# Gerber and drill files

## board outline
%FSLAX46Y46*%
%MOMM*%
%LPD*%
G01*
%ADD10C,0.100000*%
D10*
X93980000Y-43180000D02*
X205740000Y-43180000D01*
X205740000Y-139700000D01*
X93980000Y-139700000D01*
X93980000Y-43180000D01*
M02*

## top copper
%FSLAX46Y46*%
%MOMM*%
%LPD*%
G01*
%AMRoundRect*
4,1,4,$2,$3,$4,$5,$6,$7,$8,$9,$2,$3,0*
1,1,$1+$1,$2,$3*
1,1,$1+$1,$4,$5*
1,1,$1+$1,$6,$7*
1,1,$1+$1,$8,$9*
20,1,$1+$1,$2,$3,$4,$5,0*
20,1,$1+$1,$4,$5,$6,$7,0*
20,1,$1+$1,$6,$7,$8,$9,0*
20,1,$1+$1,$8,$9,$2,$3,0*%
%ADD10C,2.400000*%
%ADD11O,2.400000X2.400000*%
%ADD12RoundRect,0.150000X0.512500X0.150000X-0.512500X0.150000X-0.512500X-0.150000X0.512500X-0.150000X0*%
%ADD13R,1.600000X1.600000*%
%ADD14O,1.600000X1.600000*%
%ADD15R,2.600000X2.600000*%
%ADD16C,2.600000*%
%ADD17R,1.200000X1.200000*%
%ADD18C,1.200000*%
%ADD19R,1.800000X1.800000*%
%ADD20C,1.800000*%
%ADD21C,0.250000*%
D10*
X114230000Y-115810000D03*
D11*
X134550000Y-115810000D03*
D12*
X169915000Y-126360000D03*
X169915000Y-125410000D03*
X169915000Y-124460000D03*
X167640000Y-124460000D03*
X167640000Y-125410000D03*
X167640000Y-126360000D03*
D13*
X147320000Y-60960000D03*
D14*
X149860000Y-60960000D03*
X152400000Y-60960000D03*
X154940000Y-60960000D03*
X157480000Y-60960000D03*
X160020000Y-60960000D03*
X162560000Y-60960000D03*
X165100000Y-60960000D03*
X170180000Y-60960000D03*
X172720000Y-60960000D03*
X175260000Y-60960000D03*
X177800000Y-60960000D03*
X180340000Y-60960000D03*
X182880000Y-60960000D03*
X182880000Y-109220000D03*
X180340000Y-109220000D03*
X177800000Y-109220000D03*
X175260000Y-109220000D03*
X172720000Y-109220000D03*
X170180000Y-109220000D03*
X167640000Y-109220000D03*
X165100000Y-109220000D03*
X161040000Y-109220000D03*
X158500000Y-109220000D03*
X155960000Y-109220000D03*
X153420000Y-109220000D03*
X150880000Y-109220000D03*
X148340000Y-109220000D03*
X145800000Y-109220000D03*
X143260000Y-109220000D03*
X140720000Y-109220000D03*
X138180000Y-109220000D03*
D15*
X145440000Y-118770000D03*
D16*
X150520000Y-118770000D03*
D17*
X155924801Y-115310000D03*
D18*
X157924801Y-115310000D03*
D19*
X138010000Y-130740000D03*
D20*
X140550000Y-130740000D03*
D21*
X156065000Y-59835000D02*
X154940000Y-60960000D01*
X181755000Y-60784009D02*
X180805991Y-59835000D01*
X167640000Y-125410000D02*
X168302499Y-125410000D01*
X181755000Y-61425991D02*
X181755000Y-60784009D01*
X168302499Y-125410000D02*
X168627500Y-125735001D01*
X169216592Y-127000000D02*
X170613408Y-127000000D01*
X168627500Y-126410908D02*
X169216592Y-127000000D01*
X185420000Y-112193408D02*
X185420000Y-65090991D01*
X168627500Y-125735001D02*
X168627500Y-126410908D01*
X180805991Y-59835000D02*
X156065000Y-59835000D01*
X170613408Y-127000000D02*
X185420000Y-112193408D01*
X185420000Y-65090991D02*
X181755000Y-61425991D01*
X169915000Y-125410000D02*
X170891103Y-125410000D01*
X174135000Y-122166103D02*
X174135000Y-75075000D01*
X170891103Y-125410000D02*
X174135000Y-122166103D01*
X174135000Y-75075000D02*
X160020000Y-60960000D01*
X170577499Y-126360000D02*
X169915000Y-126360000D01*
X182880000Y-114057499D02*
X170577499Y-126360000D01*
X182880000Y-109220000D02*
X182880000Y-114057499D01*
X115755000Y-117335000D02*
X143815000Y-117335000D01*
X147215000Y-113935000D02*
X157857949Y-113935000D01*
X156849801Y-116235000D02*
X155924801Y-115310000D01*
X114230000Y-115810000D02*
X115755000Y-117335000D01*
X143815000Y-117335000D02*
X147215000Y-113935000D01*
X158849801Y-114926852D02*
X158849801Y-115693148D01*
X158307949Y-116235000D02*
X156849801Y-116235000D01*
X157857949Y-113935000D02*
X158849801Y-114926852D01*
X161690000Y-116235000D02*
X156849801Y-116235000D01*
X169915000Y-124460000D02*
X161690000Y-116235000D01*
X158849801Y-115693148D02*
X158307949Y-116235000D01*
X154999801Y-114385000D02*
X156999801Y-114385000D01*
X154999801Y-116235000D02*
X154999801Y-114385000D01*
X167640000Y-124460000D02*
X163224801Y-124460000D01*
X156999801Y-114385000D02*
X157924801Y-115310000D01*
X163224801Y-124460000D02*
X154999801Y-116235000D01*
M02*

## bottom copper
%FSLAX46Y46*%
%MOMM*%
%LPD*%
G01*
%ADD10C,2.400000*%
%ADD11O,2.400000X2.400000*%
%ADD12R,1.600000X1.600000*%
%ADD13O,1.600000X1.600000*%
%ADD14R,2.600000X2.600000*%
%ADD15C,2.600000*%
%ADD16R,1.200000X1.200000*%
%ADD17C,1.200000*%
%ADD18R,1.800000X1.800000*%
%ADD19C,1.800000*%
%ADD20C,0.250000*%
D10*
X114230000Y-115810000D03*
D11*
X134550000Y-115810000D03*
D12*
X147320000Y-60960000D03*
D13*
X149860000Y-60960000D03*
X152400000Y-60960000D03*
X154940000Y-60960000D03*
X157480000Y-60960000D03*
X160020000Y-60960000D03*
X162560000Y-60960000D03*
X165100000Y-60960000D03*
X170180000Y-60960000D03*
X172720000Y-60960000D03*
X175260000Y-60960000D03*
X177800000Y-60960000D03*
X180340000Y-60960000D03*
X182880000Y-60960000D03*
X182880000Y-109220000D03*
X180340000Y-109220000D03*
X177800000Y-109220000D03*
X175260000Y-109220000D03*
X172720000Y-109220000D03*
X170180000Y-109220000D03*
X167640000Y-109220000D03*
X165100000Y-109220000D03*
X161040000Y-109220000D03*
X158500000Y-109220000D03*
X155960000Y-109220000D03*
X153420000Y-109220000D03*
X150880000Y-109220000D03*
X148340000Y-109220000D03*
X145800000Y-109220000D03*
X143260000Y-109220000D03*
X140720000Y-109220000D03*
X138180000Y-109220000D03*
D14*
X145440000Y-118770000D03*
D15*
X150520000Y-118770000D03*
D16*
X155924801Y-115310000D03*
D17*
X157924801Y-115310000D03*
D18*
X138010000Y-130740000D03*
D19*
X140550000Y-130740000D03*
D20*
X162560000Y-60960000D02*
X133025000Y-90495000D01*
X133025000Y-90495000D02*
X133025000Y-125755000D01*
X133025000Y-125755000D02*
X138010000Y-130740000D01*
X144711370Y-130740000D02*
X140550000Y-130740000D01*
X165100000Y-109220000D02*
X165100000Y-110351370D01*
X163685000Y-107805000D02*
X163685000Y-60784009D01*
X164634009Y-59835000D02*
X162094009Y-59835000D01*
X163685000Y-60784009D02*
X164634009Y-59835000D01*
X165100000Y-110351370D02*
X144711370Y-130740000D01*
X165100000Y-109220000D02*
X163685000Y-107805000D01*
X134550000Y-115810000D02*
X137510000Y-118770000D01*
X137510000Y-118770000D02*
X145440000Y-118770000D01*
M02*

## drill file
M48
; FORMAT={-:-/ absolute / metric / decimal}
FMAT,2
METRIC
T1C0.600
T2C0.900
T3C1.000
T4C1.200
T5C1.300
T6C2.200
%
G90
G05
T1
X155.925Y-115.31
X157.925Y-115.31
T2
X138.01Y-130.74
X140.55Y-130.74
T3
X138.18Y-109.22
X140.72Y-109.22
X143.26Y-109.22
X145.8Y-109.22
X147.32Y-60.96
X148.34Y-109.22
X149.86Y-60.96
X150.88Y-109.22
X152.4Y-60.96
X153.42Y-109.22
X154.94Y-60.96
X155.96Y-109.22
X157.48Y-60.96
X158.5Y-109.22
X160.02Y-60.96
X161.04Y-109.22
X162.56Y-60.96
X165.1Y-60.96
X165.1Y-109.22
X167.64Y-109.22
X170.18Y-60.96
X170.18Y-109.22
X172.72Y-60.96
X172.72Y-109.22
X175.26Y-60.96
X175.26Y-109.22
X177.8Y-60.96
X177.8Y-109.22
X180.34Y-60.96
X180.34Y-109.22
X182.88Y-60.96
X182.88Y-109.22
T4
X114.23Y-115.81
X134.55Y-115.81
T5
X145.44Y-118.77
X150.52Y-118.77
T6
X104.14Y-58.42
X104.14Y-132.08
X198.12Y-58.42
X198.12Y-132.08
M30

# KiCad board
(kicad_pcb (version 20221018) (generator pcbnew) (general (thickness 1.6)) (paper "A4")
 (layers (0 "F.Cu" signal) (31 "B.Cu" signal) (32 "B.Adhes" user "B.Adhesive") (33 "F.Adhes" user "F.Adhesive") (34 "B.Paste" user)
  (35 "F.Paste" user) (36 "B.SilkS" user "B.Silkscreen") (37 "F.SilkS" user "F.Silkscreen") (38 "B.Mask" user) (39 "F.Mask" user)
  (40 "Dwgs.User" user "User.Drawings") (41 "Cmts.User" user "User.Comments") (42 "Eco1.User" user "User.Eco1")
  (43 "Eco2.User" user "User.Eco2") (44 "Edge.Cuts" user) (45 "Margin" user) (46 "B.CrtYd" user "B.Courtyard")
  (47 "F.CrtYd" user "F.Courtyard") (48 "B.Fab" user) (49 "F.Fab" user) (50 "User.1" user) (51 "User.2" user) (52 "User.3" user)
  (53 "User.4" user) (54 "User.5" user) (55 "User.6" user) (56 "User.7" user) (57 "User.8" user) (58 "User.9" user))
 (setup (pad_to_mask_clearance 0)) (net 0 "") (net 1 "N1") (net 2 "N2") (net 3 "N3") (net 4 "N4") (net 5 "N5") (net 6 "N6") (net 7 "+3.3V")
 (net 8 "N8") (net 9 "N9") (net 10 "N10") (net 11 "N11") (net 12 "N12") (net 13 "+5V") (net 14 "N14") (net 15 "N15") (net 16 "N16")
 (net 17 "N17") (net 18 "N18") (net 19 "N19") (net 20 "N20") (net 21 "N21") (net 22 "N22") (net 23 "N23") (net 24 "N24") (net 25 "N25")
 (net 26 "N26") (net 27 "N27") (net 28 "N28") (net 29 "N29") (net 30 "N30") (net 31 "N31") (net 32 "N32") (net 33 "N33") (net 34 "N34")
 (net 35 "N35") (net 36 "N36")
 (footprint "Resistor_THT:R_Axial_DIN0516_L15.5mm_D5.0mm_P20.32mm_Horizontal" (layer "F.Cu") (at 114.23 115.81)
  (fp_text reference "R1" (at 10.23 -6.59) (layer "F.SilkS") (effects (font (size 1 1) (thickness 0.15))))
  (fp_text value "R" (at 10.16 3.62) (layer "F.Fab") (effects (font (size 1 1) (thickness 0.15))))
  (pad "1" thru_hole circle (at 0 0) (size 2.4 2.4) (drill 1.2) (layers "*.Cu" "*.Mask") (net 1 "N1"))
  (pad "2" thru_hole oval (at 20.32 0) (size 2.4 2.4) (drill 1.2) (layers "*.Cu" "*.Mask") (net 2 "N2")))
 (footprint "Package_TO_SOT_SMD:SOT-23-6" (layer "F.Cu") (at 168.7775 125.41 180)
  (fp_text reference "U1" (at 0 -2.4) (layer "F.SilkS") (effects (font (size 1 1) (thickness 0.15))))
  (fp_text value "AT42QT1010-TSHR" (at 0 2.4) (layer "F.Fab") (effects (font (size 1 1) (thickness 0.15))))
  (pad "1" smd roundrect (at -1.1375 -0.95 180) (size 1.325 0.6) (layers "F.Cu" "F.Paste" "F.Mask") (roundrect_rratio 0.25) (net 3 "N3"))
  (pad "2" smd roundrect (at -1.1375 0 180) (size 1.325 0.6) (layers "F.Cu" "F.Paste" "F.Mask") (roundrect_rratio 0.25) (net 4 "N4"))
  (pad "3" smd roundrect (at -1.1375 0.95 180) (size 1.325 0.6) (layers "F.Cu" "F.Paste" "F.Mask") (roundrect_rratio 0.25) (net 1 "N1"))
  (pad "4" smd roundrect (at 1.1375 0.95 180) (size 1.325 0.6) (layers "F.Cu" "F.Paste" "F.Mask") (roundrect_rratio 0.25) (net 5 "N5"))
  (pad "5" smd roundrect (at 1.1375 0 180) (size 1.325 0.6) (layers "F.Cu" "F.Paste" "F.Mask") (roundrect_rratio 0.25) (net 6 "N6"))
  (pad "6" smd roundrect (at 1.1375 -0.95 180) (size 1.325 0.6) (layers "F.Cu" "F.Paste" "F.Mask") (roundrect_rratio 0.25) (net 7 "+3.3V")))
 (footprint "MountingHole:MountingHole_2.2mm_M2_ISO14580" (layer "F.Cu") (at 104.14 58.42)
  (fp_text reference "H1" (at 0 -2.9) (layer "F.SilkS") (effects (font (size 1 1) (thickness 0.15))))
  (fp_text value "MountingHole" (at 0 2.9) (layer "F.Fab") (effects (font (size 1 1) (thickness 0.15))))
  (pad "" np_thru_hole circle (at 0 0) (size 2.2 2.2) (drill 2.2) (layers "*.Cu" "*.Mask")))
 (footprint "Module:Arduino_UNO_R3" (layer "F.Cu") (at 147.32 60.96)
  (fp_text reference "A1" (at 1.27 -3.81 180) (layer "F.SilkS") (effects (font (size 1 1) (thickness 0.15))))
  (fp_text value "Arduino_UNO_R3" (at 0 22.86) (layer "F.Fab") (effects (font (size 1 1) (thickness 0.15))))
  (pad "1" thru_hole rect (at 0 0 90) (size 1.6 1.6) (drill 1) (layers "*.Cu" "*.Mask") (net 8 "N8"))
  (pad "2" thru_hole oval (at 2.54 0 90) (size 1.6 1.6) (drill 1) (layers "*.Cu" "*.Mask") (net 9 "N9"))
  (pad "3" thru_hole oval (at 5.08 0 90) (size 1.6 1.6) (drill 1) (layers "*.Cu" "*.Mask") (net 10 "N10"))
  (pad "4" thru_hole oval (at 7.62 0 90) (size 1.6 1.6) (drill 1) (layers "*.Cu" "*.Mask") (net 6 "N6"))
  (pad "5" thru_hole oval (at 10.16 0 90) (size 1.6 1.6) (drill 1) (layers "*.Cu" "*.Mask") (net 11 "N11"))
  (pad "6" thru_hole oval (at 12.7 0 90) (size 1.6 1.6) (drill 1) (layers "*.Cu" "*.Mask") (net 4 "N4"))
  (pad "7" thru_hole oval (at 15.24 0 90) (size 1.6 1.6) (drill 1) (layers "*.Cu" "*.Mask") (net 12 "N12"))
  (pad "8" thru_hole oval (at 17.78 0 90) (size 1.6 1.6) (drill 1) (layers "*.Cu" "*.Mask") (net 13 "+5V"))
  (pad "9" thru_hole oval (at 22.86 0 90) (size 1.6 1.6) (drill 1) (layers "*.Cu" "*.Mask") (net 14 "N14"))
  (pad "10" thru_hole oval (at 25.4 0 90) (size 1.6 1.6) (drill 1) (layers "*.Cu" "*.Mask") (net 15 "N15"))
  (pad "11" thru_hole oval (at 27.94 0 90) (size 1.6 1.6) (drill 1) (layers "*.Cu" "*.Mask") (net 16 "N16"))
  (pad "12" thru_hole oval (at 30.48 0 90) (size 1.6 1.6) (drill 1) (layers "*.Cu" "*.Mask") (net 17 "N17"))
  (pad "13" thru_hole oval (at 33.02 0 90) (size 1.6 1.6) (drill 1) (layers "*.Cu" "*.Mask") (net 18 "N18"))
  (pad "14" thru_hole oval (at 35.56 0 90) (size 1.6 1.6) (drill 1) (layers "*.Cu" "*.Mask") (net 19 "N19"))
  (pad "15" thru_hole oval (at 35.56 48.26 90) (size 1.6 1.6) (drill 1) (layers "*.Cu" "*.Mask") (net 3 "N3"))
  (pad "16" thru_hole oval (at 33.02 48.26 90) (size 1.6 1.6) (drill 1) (layers "*.Cu" "*.Mask") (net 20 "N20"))
  (pad "17" thru_hole oval (at 30.48 48.26 90) (size 1.6 1.6) (drill 1) (layers "*.Cu" "*.Mask") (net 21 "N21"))
  (pad "18" thru_hole oval (at 27.94 48.26 90) (size 1.6 1.6) (drill 1) (layers "*.Cu" "*.Mask") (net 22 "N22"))
  (pad "19" thru_hole oval (at 25.4 48.26 90) (size 1.6 1.6) (drill 1) (layers "*.Cu" "*.Mask") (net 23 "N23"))
  (pad "20" thru_hole oval (at 22.86 48.26 90) (size 1.6 1.6) (drill 1) (layers "*.Cu" "*.Mask") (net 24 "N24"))
  (pad "21" thru_hole oval (at 20.32 48.26 90) (size 1.6 1.6) (drill 1) (layers "*.Cu" "*.Mask") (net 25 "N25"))
  (pad "22" thru_hole oval (at 17.78 48.26 90) (size 1.6 1.6) (drill 1) (layers "*.Cu" "*.Mask") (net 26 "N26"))
  (pad "23" thru_hole oval (at 13.72 48.26 90) (size 1.6 1.6) (drill 1) (layers "*.Cu" "*.Mask") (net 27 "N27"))
  (pad "24" thru_hole oval (at 11.18 48.26 90) (size 1.6 1.6) (drill 1) (layers "*.Cu" "*.Mask") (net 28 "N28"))
  (pad "25" thru_hole oval (at 8.64 48.26 90) (size 1.6 1.6) (drill 1) (layers "*.Cu" "*.Mask") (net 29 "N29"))
  (pad "26" thru_hole oval (at 6.1 48.26 90) (size 1.6 1.6) (drill 1) (layers "*.Cu" "*.Mask") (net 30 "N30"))
  (pad "27" thru_hole oval (at 3.56 48.26 90) (size 1.6 1.6) (drill 1) (layers "*.Cu" "*.Mask") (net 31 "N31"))
  (pad "28" thru_hole oval (at 1.02 48.26 90) (size 1.6 1.6) (drill 1) (layers "*.Cu" "*.Mask") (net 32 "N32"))
  (pad "29" thru_hole oval (at -1.52 48.26 90) (size 1.6 1.6) (drill 1) (layers "*.Cu" "*.Mask") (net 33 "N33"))
  (pad "30" thru_hole oval (at -4.06 48.26 90) (size 1.6 1.6) (drill 1) (layers "*.Cu" "*.Mask") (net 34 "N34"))
  (pad "31" thru_hole oval (at -6.6 48.26 90) (size 1.6 1.6) (drill 1) (layers "*.Cu" "*.Mask") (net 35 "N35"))
  (pad "32" thru_hole oval (at -9.14 48.26 90) (size 1.6 1.6) (drill 1) (layers "*.Cu" "*.Mask") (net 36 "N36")))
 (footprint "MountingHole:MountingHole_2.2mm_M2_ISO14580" (layer "F.Cu") (at 198.12 58.42)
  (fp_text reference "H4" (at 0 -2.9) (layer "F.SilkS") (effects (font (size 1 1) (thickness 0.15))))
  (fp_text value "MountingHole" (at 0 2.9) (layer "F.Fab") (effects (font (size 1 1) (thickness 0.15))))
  (pad "" np_thru_hole circle (at 0 0) (size 2.2 2.2) (drill 2.2) (layers "*.Cu" "*.Mask")))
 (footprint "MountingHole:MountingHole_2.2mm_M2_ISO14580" (layer "F.Cu") (at 198.12 132.08)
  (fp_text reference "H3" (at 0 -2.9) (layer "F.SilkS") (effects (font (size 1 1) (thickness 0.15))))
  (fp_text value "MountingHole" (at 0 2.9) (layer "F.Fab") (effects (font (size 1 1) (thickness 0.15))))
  (pad "" np_thru_hole circle (at 0 0) (size 2.2 2.2) (drill 2.2) (layers "*.Cu" "*.Mask")))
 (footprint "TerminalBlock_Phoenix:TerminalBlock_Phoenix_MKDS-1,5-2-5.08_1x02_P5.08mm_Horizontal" (layer "F.Cu") (at 145.44 118.77)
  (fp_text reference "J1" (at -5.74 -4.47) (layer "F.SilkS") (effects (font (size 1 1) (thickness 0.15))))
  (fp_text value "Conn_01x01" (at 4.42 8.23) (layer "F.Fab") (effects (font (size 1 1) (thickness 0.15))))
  (pad "1" thru_hole rect (at 0 0) (size 2.6 2.6) (drill 1.3) (layers "*.Cu" "*.Mask") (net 2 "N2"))
  (pad "2" thru_hole circle (at 5.08 0) (size 2.6 2.6) (drill 1.3) (layers "*.Cu" "*.Mask")))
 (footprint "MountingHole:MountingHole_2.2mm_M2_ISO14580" (layer "F.Cu") (at 104.14 132.08)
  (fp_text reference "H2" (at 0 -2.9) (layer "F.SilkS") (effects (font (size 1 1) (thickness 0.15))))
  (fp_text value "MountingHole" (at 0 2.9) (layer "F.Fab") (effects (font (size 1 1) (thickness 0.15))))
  (pad "" np_thru_hole circle (at 0 0) (size 2.2 2.2) (drill 2.2) (layers "*.Cu" "*.Mask")))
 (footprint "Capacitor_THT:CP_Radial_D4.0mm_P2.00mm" (layer "F.Cu") (at 155.924801 115.31)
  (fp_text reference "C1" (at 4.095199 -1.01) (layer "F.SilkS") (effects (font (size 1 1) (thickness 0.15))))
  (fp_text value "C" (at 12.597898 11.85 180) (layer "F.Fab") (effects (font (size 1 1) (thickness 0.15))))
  (pad "1" thru_hole rect (at 0 0) (size 1.2 1.2) (drill 0.6) (layers "*.Cu" "*.Mask") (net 1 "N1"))
  (pad "2" thru_hole circle (at 2 0) (size 1.2 1.2) (drill 0.6) (layers "*.Cu" "*.Mask") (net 5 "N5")))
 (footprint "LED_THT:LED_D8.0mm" (layer "F.Cu") (at 138.01 130.74)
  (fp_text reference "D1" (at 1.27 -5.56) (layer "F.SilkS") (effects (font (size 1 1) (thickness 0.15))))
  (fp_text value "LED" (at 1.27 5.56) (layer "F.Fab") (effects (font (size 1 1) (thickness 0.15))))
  (pad "1" thru_hole rect (at 0 0) (size 1.8 1.8) (drill 0.9) (layers "*.Cu" "*.Mask") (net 12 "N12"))
  (pad "2" thru_hole circle (at 2.54 0) (size 1.8 1.8) (drill 0.9) (layers "*.Cu" "*.Mask") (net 26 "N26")))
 (gr_rect (start 93.98 43.18) (end 205.74 139.7) (stroke (width 0.1) (type default)) (fill none) (layer "Edge.Cuts"))
 (segment (start 156.065 59.835) (end 154.94 60.96) (width 0.25) (layer "F.Cu") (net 6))
 (segment (start 181.755 60.784009) (end 180.805991 59.835) (width 0.25) (layer "F.Cu") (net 6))
 (segment (start 167.64 125.41) (end 168.302499 125.41) (width 0.25) (layer "F.Cu") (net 6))
 (segment (start 181.755 61.425991) (end 181.755 60.784009) (width 0.25) (layer "F.Cu") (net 6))
 (segment (start 168.302499 125.41) (end 168.6275 125.735001) (width 0.25) (layer "F.Cu") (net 6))
 (segment (start 169.216592 127) (end 170.613408 127) (width 0.25) (layer "F.Cu") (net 6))
 (segment (start 168.6275 126.410908) (end 169.216592 127) (width 0.25) (layer "F.Cu") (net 6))
 (segment (start 185.42 112.193408) (end 185.42 65.090991) (width 0.25) (layer "F.Cu") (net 6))
 (segment (start 168.6275 125.735001) (end 168.6275 126.410908) (width 0.25) (layer "F.Cu") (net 6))
 (segment (start 180.805991 59.835) (end 156.065 59.835) (width 0.25) (layer "F.Cu") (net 6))
 (segment (start 170.613408 127) (end 185.42 112.193408) (width 0.25) (layer "F.Cu") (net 6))
 (segment (start 185.42 65.090991) (end 181.755 61.425991) (width 0.25) (layer "F.Cu") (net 6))
 (segment (start 169.915 125.41) (end 170.891103 125.41) (width 0.25) (layer "F.Cu") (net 4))
 (segment (start 174.135 122.166103) (end 174.135 75.075) (width 0.25) (layer "F.Cu") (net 4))
 (segment (start 170.891103 125.41) (end 174.135 122.166103) (width 0.25) (layer "F.Cu") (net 4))
 (segment (start 174.135 75.075) (end 160.02 60.96) (width 0.25) (layer "F.Cu") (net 4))
 (segment (start 162.56 60.96) (end 133.025 90.495) (width 0.25) (layer "B.Cu") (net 12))
 (segment (start 133.025 90.495) (end 133.025 125.755) (width 0.25) (layer "B.Cu") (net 12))
 (segment (start 133.025 125.755) (end 138.01 130.74) (width 0.25) (layer "B.Cu") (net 12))
 (segment (start 170.577499 126.36) (end 169.915 126.36) (width 0.25) (layer "F.Cu") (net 3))
 (segment (start 182.88 114.057499) (end 170.577499 126.36) (width 0.25) (layer "F.Cu") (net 3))
 (segment (start 182.88 109.22) (end 182.88 114.057499) (width 0.25) (layer "F.Cu") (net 3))
 (segment (start 144.71137 130.74) (end 140.55 130.74) (width 0.25) (layer "B.Cu") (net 26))
 (segment (start 165.1 109.22) (end 165.1 110.35137) (width 0.25) (layer "B.Cu") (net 26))
 (segment (start 163.685 107.805) (end 163.685 60.784009) (width 0.25) (layer "B.Cu") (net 26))
 (segment (start 164.634009 59.835) (end 162.094009 59.835) (width 0.25) (layer "B.Cu") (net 26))
 (segment (start 163.685 60.784009) (end 164.634009 59.835) (width 0.25) (layer "B.Cu") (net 26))
 (segment (start 165.1 110.35137) (end 144.71137 130.74) (width 0.25) (layer "B.Cu") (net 26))
 (segment (start 165.1 109.22) (end 163.685 107.805) (width 0.25) (layer "B.Cu") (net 26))
 (segment (start 115.755 117.335) (end 143.815 117.335) (width 0.25) (layer "F.Cu") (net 1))
 (segment (start 147.215 113.935) (end 157.857949 113.935) (width 0.25) (layer "F.Cu") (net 1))
 (segment (start 156.849801 116.235) (end 155.924801 115.31) (width 0.25) (layer "F.Cu") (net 1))
 (segment (start 114.23 115.81) (end 115.755 117.335) (width 0.25) (layer "F.Cu") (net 1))
 (segment (start 143.815 117.335) (end 147.215 113.935) (width 0.25) (layer "F.Cu") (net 1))
 (segment (start 158.849801 114.926852) (end 158.849801 115.693148) (width 0.25) (layer "F.Cu") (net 1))
 (segment (start 158.307949 116.235) (end 156.849801 116.235) (width 0.25) (layer "F.Cu") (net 1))
 (segment (start 157.857949 113.935) (end 158.849801 114.926852) (width 0.25) (layer "F.Cu") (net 1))
 (segment (start 161.69 116.235) (end 156.849801 116.235) (width 0.25) (layer "F.Cu") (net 1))
 (segment (start 169.915 124.46) (end 161.69 116.235) (width 0.25) (layer "F.Cu") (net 1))
 (segment (start 158.849801 115.693148) (end 158.307949 116.235) (width 0.25) (layer "F.Cu") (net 1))
 (segment (start 154.999801 114.385) (end 156.999801 114.385) (width 0.25) (layer "F.Cu") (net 5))
 (segment (start 154.999801 116.235) (end 154.999801 114.385) (width 0.25) (layer "F.Cu") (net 5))
 (segment (start 167.64 124.46) (end 163.224801 124.46) (width 0.25) (layer "F.Cu") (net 5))
 (segment (start 156.999801 114.385) (end 157.924801 115.31) (width 0.25) (layer "F.Cu") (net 5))
 (segment (start 163.224801 124.46) (end 154.999801 116.235) (width 0.25) (layer "F.Cu") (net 5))
 (segment (start 134.55 115.81) (end 137.51 118.77) (width 0.25) (layer "B.Cu") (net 2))
 (segment (start 137.51 118.77) (end 145.44 118.77) (width 0.25) (layer "B.Cu") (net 2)))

